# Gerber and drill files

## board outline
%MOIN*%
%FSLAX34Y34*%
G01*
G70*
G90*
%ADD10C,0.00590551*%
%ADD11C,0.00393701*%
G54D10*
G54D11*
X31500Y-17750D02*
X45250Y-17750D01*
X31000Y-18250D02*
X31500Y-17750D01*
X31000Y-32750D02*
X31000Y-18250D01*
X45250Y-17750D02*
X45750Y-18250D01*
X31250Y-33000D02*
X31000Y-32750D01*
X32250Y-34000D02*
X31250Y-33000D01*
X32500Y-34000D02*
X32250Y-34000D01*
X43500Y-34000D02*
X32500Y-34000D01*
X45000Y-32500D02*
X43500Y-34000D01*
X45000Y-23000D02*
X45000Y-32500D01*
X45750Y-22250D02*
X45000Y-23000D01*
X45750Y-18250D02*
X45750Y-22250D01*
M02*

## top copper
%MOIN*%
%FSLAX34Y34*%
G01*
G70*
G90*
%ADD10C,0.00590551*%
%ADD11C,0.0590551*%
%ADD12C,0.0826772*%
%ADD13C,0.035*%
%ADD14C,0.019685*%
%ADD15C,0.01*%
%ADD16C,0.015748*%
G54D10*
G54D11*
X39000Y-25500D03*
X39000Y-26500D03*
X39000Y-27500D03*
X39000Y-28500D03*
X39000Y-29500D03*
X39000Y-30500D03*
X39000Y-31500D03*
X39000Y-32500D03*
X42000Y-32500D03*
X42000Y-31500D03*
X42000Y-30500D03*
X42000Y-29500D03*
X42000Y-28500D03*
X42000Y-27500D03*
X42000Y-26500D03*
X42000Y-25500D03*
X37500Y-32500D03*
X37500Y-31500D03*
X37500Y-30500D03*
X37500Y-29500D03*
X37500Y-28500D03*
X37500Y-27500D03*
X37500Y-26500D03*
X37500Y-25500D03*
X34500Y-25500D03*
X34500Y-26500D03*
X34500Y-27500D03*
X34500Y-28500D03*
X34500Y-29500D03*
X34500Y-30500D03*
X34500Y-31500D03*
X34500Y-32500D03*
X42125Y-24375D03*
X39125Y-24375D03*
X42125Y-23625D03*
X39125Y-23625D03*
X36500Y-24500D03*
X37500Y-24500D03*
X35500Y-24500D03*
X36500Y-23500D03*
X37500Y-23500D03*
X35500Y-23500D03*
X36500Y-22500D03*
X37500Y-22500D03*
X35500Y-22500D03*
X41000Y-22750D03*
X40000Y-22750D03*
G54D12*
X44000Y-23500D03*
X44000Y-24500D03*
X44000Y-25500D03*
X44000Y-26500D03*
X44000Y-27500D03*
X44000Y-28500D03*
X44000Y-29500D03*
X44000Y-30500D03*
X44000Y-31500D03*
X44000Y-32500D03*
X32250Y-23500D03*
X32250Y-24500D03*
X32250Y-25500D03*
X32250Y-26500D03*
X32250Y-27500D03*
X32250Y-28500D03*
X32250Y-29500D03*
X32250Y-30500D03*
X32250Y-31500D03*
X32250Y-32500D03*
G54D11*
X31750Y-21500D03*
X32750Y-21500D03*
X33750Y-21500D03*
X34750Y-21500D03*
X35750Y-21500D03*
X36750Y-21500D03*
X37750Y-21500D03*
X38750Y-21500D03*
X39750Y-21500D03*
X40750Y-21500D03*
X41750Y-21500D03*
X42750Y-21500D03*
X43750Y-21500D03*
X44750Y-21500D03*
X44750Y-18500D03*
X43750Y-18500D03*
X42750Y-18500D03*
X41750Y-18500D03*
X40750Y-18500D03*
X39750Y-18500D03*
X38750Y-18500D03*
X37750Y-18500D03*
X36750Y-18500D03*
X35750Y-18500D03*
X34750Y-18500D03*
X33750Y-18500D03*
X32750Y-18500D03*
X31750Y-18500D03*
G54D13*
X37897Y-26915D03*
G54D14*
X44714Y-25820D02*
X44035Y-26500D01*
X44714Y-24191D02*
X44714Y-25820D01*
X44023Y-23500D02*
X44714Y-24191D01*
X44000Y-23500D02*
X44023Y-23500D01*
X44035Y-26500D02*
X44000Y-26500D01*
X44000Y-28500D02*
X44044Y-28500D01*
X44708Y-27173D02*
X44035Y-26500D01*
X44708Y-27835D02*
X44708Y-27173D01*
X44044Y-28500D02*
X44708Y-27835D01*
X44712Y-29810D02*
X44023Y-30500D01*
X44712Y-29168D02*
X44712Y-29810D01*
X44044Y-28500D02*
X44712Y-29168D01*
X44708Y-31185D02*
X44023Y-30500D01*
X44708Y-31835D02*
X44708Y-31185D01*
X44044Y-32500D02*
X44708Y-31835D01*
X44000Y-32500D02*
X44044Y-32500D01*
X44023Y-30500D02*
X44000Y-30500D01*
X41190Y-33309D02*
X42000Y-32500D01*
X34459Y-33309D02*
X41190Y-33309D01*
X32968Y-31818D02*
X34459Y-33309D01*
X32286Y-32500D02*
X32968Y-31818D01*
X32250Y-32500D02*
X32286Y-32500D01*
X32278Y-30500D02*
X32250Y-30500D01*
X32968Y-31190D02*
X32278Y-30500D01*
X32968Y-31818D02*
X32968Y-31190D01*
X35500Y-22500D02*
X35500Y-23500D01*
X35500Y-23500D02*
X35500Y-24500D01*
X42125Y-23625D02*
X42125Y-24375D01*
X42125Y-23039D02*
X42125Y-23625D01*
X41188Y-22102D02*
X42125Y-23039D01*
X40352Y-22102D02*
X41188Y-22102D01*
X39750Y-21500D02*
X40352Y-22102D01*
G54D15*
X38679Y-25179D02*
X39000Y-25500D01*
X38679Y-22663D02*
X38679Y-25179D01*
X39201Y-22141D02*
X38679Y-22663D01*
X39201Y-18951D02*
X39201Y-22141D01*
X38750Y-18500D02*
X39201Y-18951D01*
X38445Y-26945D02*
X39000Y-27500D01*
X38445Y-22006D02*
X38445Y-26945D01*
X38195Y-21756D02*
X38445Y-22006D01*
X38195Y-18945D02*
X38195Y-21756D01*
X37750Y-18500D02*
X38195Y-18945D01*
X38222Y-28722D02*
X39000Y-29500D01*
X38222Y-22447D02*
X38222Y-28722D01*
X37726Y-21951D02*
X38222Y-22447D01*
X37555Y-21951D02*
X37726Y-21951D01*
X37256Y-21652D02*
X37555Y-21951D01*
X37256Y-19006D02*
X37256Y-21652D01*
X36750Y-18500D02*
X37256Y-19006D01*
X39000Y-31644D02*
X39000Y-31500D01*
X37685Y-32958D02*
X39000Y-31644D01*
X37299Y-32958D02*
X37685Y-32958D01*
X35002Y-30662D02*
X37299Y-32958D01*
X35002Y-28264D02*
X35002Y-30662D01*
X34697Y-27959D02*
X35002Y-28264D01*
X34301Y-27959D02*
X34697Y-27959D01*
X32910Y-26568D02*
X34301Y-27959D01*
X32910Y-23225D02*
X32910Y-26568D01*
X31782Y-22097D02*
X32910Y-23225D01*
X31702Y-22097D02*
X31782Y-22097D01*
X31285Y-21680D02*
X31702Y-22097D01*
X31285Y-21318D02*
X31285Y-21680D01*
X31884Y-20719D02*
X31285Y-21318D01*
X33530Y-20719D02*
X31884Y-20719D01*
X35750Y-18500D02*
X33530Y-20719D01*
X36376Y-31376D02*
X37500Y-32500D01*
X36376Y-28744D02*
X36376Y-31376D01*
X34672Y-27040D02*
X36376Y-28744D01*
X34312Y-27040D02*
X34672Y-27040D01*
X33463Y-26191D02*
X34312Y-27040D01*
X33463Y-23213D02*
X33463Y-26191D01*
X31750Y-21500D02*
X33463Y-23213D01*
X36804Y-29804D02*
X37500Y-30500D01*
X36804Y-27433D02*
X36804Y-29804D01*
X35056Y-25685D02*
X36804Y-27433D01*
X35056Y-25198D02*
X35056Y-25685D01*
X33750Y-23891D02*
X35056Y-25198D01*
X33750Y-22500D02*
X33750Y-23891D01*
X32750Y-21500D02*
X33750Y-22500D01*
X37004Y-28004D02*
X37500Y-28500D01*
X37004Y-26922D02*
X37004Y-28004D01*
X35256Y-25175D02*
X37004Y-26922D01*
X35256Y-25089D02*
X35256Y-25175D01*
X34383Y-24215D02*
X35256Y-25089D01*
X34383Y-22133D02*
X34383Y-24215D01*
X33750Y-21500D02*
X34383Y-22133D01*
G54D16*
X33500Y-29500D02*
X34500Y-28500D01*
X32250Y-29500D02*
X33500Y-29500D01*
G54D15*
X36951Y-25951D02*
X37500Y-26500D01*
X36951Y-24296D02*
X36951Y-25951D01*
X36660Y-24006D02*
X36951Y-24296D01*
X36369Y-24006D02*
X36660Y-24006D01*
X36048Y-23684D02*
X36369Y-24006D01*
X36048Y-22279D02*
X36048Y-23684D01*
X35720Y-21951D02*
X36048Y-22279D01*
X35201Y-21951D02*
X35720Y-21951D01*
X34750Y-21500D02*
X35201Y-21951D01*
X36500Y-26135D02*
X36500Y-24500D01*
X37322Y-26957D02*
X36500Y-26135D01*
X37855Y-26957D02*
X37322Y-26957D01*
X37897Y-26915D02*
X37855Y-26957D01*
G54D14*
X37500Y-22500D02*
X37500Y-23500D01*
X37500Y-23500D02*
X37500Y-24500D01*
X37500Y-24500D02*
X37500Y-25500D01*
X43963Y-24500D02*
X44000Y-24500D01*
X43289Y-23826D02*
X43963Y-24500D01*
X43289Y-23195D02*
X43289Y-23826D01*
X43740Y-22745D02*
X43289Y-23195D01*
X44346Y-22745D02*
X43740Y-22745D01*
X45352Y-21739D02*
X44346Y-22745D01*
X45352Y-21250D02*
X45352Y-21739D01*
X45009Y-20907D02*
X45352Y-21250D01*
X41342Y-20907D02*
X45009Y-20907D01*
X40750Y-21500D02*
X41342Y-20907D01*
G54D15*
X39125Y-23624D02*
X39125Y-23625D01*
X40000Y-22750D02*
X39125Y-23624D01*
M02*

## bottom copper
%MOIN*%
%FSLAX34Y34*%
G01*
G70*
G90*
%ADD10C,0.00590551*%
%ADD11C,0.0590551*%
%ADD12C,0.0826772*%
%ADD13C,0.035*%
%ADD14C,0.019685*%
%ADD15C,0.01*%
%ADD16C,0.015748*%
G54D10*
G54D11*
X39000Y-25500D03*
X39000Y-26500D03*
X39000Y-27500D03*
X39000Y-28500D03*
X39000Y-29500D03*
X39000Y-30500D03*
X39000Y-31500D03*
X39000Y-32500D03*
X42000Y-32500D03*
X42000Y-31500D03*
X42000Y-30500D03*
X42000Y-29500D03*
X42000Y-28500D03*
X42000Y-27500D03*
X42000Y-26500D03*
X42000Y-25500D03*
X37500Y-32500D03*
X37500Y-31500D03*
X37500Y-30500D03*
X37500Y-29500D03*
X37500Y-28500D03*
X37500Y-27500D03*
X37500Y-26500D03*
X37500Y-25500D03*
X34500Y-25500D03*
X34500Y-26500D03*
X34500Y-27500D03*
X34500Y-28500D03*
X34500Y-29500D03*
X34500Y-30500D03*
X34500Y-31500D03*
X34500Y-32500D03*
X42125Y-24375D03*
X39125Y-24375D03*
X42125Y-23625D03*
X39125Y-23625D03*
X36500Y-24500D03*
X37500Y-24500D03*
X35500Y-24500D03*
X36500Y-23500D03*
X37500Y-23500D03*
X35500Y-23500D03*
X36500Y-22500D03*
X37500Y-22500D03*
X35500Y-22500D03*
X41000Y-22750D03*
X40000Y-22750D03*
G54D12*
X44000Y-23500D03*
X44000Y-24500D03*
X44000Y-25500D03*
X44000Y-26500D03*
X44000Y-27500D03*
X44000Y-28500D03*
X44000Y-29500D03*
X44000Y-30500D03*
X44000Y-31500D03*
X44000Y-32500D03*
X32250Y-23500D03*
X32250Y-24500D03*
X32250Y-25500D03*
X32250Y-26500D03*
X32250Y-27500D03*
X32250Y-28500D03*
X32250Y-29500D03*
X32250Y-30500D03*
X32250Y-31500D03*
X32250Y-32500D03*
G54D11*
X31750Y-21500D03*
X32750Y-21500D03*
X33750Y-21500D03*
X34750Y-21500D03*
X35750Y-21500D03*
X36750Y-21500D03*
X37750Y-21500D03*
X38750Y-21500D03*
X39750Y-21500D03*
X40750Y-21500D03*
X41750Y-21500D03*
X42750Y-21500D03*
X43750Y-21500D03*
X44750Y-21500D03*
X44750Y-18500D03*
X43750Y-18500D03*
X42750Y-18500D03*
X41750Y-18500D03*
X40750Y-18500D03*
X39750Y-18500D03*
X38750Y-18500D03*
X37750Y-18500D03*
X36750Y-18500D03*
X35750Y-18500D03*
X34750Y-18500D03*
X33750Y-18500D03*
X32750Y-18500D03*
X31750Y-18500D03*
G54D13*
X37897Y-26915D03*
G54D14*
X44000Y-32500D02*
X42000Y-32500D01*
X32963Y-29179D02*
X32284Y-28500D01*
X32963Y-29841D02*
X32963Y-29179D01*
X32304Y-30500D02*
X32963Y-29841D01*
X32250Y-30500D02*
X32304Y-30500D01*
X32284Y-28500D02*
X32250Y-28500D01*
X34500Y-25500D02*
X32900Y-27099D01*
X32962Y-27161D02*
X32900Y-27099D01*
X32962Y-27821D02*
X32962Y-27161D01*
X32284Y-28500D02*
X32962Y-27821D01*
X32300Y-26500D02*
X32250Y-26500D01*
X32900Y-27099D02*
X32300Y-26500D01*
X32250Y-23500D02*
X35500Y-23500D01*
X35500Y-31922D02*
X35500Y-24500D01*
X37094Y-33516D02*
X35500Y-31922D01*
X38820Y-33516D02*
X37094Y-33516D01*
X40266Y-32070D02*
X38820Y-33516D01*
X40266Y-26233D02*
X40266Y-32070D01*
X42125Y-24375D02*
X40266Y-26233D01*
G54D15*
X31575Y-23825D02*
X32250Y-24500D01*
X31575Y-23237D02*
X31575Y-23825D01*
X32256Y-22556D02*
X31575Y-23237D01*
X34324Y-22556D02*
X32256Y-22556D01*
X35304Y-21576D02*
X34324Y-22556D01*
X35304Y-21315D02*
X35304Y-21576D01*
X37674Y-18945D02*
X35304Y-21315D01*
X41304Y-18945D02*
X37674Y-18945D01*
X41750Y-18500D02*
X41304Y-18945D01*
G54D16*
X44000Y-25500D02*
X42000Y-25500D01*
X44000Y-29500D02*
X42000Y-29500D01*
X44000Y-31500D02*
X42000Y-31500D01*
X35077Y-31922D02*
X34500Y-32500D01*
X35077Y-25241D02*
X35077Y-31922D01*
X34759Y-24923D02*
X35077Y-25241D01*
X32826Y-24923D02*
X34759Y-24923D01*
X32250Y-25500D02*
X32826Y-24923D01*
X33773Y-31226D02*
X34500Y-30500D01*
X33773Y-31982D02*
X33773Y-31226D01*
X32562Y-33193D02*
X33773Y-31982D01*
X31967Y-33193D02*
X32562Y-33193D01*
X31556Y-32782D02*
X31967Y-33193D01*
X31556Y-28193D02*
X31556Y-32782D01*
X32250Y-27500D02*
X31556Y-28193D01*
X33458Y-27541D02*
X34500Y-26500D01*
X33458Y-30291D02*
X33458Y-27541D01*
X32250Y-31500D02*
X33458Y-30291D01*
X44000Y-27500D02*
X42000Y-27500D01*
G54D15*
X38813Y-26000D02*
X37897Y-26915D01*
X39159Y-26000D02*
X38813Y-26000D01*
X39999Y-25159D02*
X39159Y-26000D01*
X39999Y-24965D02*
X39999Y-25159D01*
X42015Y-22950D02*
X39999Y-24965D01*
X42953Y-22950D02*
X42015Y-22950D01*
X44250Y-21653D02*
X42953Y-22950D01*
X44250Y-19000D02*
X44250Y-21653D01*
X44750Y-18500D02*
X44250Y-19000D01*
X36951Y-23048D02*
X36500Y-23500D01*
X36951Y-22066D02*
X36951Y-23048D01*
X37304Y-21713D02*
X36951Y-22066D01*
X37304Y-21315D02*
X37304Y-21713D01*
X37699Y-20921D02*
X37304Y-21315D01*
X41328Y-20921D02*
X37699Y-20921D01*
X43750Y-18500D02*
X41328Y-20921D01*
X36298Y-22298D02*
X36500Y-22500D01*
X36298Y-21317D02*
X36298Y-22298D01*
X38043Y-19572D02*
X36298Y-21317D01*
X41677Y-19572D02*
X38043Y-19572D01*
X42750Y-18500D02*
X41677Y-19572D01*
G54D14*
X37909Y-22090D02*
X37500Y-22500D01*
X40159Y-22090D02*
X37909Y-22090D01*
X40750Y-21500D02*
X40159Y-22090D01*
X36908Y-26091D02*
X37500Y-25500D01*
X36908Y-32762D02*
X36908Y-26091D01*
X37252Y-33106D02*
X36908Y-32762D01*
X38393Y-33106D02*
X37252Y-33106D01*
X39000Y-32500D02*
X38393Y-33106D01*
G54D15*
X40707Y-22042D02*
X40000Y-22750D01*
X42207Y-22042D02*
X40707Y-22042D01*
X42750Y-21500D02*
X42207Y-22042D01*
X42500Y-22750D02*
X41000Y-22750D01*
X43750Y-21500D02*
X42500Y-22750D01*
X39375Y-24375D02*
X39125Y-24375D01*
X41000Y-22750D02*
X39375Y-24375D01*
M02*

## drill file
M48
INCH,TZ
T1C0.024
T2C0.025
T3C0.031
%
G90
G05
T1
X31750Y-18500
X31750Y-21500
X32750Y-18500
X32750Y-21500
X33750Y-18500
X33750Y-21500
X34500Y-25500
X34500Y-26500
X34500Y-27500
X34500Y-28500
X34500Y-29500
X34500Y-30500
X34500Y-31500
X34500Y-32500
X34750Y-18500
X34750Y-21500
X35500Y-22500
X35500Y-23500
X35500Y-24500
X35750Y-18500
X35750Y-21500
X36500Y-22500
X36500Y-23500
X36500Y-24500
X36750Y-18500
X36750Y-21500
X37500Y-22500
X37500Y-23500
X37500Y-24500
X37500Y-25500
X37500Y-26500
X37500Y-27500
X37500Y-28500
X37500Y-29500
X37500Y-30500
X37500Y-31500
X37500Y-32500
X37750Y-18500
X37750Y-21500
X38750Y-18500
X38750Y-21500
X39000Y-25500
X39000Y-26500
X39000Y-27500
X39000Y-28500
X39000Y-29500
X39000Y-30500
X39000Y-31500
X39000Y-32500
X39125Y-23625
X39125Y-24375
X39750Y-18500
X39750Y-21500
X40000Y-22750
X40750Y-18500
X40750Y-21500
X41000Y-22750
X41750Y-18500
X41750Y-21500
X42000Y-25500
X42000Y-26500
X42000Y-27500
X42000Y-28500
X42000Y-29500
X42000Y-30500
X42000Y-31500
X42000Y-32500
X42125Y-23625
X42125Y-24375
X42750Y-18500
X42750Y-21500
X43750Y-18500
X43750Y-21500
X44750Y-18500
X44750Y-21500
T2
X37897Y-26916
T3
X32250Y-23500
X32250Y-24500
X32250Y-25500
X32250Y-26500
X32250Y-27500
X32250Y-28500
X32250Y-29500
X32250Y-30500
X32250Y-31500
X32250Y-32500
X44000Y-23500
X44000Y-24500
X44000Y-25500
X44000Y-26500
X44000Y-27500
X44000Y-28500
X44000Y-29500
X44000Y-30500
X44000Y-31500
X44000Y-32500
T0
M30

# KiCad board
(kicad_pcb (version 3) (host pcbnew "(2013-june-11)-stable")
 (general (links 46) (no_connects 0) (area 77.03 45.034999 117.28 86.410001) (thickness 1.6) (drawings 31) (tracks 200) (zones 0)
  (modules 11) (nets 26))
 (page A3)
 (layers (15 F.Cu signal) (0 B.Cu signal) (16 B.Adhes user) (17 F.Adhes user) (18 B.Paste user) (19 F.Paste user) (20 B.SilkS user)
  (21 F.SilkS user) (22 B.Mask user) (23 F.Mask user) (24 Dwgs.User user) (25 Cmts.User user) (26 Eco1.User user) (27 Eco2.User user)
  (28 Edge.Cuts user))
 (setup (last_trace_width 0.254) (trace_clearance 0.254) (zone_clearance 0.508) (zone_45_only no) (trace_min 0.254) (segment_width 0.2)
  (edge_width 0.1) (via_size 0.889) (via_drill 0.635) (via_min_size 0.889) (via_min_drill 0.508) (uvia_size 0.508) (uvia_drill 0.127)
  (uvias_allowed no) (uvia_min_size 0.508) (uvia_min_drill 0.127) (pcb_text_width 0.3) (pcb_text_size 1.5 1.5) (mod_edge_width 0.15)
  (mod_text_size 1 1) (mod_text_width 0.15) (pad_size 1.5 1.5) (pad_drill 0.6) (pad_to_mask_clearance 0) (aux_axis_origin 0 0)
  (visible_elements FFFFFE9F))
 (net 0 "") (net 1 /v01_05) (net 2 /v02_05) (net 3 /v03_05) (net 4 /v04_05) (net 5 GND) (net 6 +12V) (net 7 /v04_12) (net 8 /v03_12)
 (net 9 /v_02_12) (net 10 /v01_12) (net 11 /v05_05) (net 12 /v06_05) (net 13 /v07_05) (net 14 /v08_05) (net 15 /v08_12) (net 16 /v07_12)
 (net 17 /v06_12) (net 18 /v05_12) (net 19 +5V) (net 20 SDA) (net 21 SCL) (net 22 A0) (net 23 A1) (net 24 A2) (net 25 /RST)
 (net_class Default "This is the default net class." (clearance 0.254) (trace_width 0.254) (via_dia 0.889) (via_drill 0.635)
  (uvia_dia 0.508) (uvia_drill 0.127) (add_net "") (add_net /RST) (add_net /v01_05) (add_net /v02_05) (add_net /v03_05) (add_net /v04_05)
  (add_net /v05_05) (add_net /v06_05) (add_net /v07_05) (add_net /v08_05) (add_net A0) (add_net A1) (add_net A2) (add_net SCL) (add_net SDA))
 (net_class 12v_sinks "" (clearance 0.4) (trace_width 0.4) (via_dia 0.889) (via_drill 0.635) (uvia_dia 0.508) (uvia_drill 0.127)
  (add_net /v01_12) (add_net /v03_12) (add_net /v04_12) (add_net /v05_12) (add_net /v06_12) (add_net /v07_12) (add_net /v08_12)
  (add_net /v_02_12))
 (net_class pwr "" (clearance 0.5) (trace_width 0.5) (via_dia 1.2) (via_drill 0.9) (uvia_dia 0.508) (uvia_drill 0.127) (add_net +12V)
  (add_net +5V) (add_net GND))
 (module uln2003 (layer F.Cu) (at 100.33 74.93)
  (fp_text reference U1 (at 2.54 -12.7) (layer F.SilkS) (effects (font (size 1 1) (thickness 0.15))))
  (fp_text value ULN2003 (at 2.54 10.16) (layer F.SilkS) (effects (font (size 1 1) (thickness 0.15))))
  (pad 1 thru_hole circle (at -1.27 -10.16) (size 1.5 1.5) (drill 0.6) (layers *.Cu *.Mask F.SilkS) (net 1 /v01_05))
  (pad 2 thru_hole circle (at -1.27 -7.62) (size 1.5 1.5) (drill 0.6) (layers *.Cu *.Mask F.SilkS))
  (pad 3 thru_hole circle (at -1.27 -5.08) (size 1.5 1.5) (drill 0.6) (layers *.Cu *.Mask F.SilkS) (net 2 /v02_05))
  (pad 4 thru_hole circle (at -1.27 -2.54) (size 1.5 1.5) (drill 0.6) (layers *.Cu *.Mask F.SilkS))
  (pad 5 thru_hole circle (at -1.27 0) (size 1.5 1.5) (drill 0.6) (layers *.Cu *.Mask F.SilkS) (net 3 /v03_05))
  (pad 6 thru_hole circle (at -1.27 2.54) (size 1.5 1.5) (drill 0.6) (layers *.Cu *.Mask F.SilkS))
  (pad 7 thru_hole circle (at -1.27 5.08) (size 1.5 1.5) (drill 0.6) (layers *.Cu *.Mask F.SilkS) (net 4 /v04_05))
  (pad 8 thru_hole circle (at -1.27 7.62) (size 1.5 1.5) (drill 0.6) (layers *.Cu *.Mask F.SilkS) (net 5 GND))
  (pad 9 thru_hole circle (at 6.35 7.62) (size 1.5 1.5) (drill 0.6) (layers *.Cu *.Mask F.SilkS) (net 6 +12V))
  (pad 10 thru_hole circle (at 6.35 5.08) (size 1.5 1.5) (drill 0.6) (layers *.Cu *.Mask F.SilkS) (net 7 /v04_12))
  (pad 11 thru_hole circle (at 6.35 2.54) (size 1.5 1.5) (drill 0.6) (layers *.Cu *.Mask F.SilkS))
  (pad 12 thru_hole circle (at 6.35 0) (size 1.5 1.5) (drill 0.6) (layers *.Cu *.Mask F.SilkS) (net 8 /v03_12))
  (pad 13 thru_hole circle (at 6.35 -2.54) (size 1.5 1.5) (drill 0.6) (layers *.Cu *.Mask F.SilkS))
  (pad 14 thru_hole circle (at 6.35 -5.08) (size 1.5 1.5) (drill 0.6) (layers *.Cu *.Mask F.SilkS) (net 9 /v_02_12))
  (pad 15 thru_hole circle (at 6.35 -7.62) (size 1.5 1.5) (drill 0.6) (layers *.Cu *.Mask F.SilkS))
  (pad 16 thru_hole circle (at 6.35 -10.16) (size 1.5 1.5) (drill 0.6) (layers *.Cu *.Mask F.SilkS) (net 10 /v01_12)))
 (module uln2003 (layer F.Cu) (at 93.98 72.39 180)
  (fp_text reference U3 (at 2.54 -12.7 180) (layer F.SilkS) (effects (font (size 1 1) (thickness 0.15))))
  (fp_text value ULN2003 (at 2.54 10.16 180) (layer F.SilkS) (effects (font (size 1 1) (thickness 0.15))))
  (pad 1 thru_hole circle (at -1.27 -10.16 180) (size 1.5 1.5) (drill 0.6) (layers *.Cu *.Mask F.SilkS) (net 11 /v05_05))
  (pad 2 thru_hole circle (at -1.27 -7.62 180) (size 1.5 1.5) (drill 0.6) (layers *.Cu *.Mask F.SilkS))
  (pad 3 thru_hole circle (at -1.27 -5.08 180) (size 1.5 1.5) (drill 0.6) (layers *.Cu *.Mask F.SilkS) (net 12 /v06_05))
  (pad 4 thru_hole circle (at -1.27 -2.54 180) (size 1.5 1.5) (drill 0.6) (layers *.Cu *.Mask F.SilkS))
  (pad 5 thru_hole circle (at -1.27 0 180) (size 1.5 1.5) (drill 0.6) (layers *.Cu *.Mask F.SilkS) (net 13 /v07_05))
  (pad 6 thru_hole circle (at -1.27 2.54 180) (size 1.5 1.5) (drill 0.6) (layers *.Cu *.Mask F.SilkS))
  (pad 7 thru_hole circle (at -1.27 5.08 180) (size 1.5 1.5) (drill 0.6) (layers *.Cu *.Mask F.SilkS) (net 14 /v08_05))
  (pad 8 thru_hole circle (at -1.27 7.62 180) (size 1.5 1.5) (drill 0.6) (layers *.Cu *.Mask F.SilkS) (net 5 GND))
  (pad 9 thru_hole circle (at 6.35 7.62 180) (size 1.5 1.5) (drill 0.6) (layers *.Cu *.Mask F.SilkS) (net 6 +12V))
  (pad 10 thru_hole circle (at 6.35 5.08 180) (size 1.5 1.5) (drill 0.6) (layers *.Cu *.Mask F.SilkS) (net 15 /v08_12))
  (pad 11 thru_hole circle (at 6.35 2.54 180) (size 1.5 1.5) (drill 0.6) (layers *.Cu *.Mask F.SilkS))
  (pad 12 thru_hole circle (at 6.35 0 180) (size 1.5 1.5) (drill 0.6) (layers *.Cu *.Mask F.SilkS) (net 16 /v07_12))
  (pad 13 thru_hole circle (at 6.35 -2.54 180) (size 1.5 1.5) (drill 0.6) (layers *.Cu *.Mask F.SilkS))
  (pad 14 thru_hole circle (at 6.35 -5.08 180) (size 1.5 1.5) (drill 0.6) (layers *.Cu *.Mask F.SilkS) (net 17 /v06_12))
  (pad 15 thru_hole circle (at 6.35 -7.62 180) (size 1.5 1.5) (drill 0.6) (layers *.Cu *.Mask F.SilkS))
  (pad 16 thru_hole circle (at 6.35 -10.16 180) (size 1.5 1.5) (drill 0.6) (layers *.Cu *.Mask F.SilkS) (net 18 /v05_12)))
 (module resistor (layer F.Cu) (at 104.458 61.9125 180)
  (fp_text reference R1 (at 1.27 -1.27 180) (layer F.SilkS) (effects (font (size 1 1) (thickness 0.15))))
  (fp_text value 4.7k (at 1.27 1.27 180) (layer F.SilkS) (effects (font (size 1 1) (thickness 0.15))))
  (pad 1 thru_hole circle (at -2.54 0 180) (size 1.5 1.5) (drill 0.6) (layers *.Cu *.Mask F.SilkS) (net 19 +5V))
  (pad 2 thru_hole circle (at 5.08 0 180) (size 1.5 1.5) (drill 0.6) (layers *.Cu *.Mask F.SilkS) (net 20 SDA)))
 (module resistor (layer F.Cu) (at 104.458 60.0075 180)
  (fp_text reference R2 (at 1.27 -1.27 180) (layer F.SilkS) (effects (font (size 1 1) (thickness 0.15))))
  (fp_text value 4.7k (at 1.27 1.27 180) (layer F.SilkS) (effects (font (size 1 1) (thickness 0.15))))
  (pad 1 thru_hole circle (at -2.54 0 180) (size 1.5 1.5) (drill 0.6) (layers *.Cu *.Mask F.SilkS) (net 19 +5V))
  (pad 2 thru_hole circle (at 5.08 0 180) (size 1.5 1.5) (drill 0.6) (layers *.Cu *.Mask F.SilkS) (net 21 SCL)))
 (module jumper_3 (layer F.Cu) (at 92.71 62.23)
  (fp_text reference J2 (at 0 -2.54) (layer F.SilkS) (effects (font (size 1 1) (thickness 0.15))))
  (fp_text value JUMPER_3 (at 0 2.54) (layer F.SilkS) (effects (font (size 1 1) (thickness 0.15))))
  (pad 2 thru_hole circle (at 0 0) (size 1.5 1.5) (drill 0.6) (layers *.Cu *.Mask F.SilkS) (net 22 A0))
  (pad 3 thru_hole circle (at 2.54 0) (size 1.5 1.5) (drill 0.6) (layers *.Cu *.Mask F.SilkS) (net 5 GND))
  (pad 1 thru_hole circle (at -2.54 0) (size 1.5 1.5) (drill 0.6) (layers *.Cu *.Mask F.SilkS) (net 19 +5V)))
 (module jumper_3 (layer F.Cu) (at 92.71 59.69)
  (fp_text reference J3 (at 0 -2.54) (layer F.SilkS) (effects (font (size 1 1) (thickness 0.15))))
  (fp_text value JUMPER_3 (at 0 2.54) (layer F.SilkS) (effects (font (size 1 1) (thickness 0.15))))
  (pad 2 thru_hole circle (at 0 0) (size 1.5 1.5) (drill 0.6) (layers *.Cu *.Mask F.SilkS) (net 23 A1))
  (pad 3 thru_hole circle (at 2.54 0) (size 1.5 1.5) (drill 0.6) (layers *.Cu *.Mask F.SilkS) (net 5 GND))
  (pad 1 thru_hole circle (at -2.54 0) (size 1.5 1.5) (drill 0.6) (layers *.Cu *.Mask F.SilkS) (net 19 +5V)))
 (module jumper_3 (layer F.Cu) (at 92.71 57.15)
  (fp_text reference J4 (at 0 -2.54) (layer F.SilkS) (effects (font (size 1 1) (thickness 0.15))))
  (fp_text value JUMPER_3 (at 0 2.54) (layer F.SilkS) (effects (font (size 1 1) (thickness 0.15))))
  (pad 2 thru_hole circle (at 0 0) (size 1.5 1.5) (drill 0.6) (layers *.Cu *.Mask F.SilkS) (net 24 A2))
  (pad 3 thru_hole circle (at 2.54 0) (size 1.5 1.5) (drill 0.6) (layers *.Cu *.Mask F.SilkS) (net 5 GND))
  (pad 1 thru_hole circle (at -2.54 0) (size 1.5 1.5) (drill 0.6) (layers *.Cu *.Mask F.SilkS) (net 19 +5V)))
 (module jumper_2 (layer F.Cu) (at 102.87 57.785 180)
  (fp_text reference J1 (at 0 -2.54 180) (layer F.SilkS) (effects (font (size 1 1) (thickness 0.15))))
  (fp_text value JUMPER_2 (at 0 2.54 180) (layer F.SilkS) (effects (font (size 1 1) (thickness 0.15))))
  (pad 1 thru_hole circle (at -1.27 0 180) (size 1.5 1.5) (drill 0.6) (layers *.Cu *.Mask F.SilkS) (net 20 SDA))
  (pad 2 thru_hole circle (at 1.27 0 180) (size 1.5 1.5) (drill 0.6) (layers *.Cu *.Mask F.SilkS) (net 21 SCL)))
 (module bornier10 (layer F.Cu) (at 111.76 72.39 270)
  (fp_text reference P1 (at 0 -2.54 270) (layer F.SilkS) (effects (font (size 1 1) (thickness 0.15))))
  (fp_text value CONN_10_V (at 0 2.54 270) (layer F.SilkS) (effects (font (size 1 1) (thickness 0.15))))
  (pad 1 thru_hole circle (at -12.7 0 270) (size 2.1 2.1) (drill 0.8) (layers *.Cu *.Mask F.SilkS) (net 6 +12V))
  (pad 2 thru_hole circle (at -10.16 0 270) (size 2.1 2.1) (drill 0.8) (layers *.Cu *.Mask F.SilkS) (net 5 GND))
  (pad 3 thru_hole circle (at -7.62 0 270) (size 2.1 2.1) (drill 0.8) (layers *.Cu *.Mask F.SilkS) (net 10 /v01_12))
  (pad 4 thru_hole circle (at -5.08 0 270) (size 2.1 2.1) (drill 0.8) (layers *.Cu *.Mask F.SilkS) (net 6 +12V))
  (pad 5 thru_hole circle (at -2.54 0 270) (size 2.1 2.1) (drill 0.8) (layers *.Cu *.Mask F.SilkS) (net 9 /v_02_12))
  (pad 6 thru_hole circle (at 0 0 270) (size 2.1 2.1) (drill 0.8) (layers *.Cu *.Mask F.SilkS) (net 6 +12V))
  (pad 7 thru_hole circle (at 2.54 0 270) (size 2.1 2.1) (drill 0.8) (layers *.Cu *.Mask F.SilkS) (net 8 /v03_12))
  (pad 8 thru_hole circle (at 5.08 0 270) (size 2.1 2.1) (drill 0.8) (layers *.Cu *.Mask F.SilkS) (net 6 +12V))
  (pad 9 thru_hole circle (at 7.62 0 270) (size 2.1 2.1) (drill 0.8) (layers *.Cu *.Mask F.SilkS) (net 7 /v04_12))
  (pad 10 thru_hole circle (at 10.16 0 270) (size 2.1 2.1) (drill 0.8) (layers *.Cu *.Mask F.SilkS) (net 6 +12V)))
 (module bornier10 (layer F.Cu) (at 81.915 72.39 270)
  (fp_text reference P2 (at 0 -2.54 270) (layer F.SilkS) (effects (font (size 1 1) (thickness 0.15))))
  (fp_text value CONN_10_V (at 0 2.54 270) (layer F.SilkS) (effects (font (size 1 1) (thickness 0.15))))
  (pad 1 thru_hole circle (at -12.7 0 270) (size 2.1 2.1) (drill 0.8) (layers *.Cu *.Mask F.SilkS) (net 19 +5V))
  (pad 2 thru_hole circle (at -10.16 0 270) (size 2.1 2.1) (drill 0.8) (layers *.Cu *.Mask F.SilkS) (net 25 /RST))
  (pad 3 thru_hole circle (at -7.62 0 270) (size 2.1 2.1) (drill 0.8) (layers *.Cu *.Mask F.SilkS) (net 18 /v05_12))
  (pad 4 thru_hole circle (at -5.08 0 270) (size 2.1 2.1) (drill 0.8) (layers *.Cu *.Mask F.SilkS) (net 6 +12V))
  (pad 5 thru_hole circle (at -2.54 0 270) (size 2.1 2.1) (drill 0.8) (layers *.Cu *.Mask F.SilkS) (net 17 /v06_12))
  (pad 6 thru_hole circle (at 0 0 270) (size 2.1 2.1) (drill 0.8) (layers *.Cu *.Mask F.SilkS) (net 6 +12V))
  (pad 7 thru_hole circle (at 2.54 0 270) (size 2.1 2.1) (drill 0.8) (layers *.Cu *.Mask F.SilkS) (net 16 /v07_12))
  (pad 8 thru_hole circle (at 5.08 0 270) (size 2.1 2.1) (drill 0.8) (layers *.Cu *.Mask F.SilkS) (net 6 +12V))
  (pad 9 thru_hole circle (at 7.62 0 270) (size 2.1 2.1) (drill 0.8) (layers *.Cu *.Mask F.SilkS) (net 15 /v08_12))
  (pad 10 thru_hole circle (at 10.16 0 270) (size 2.1 2.1) (drill 0.8) (layers *.Cu *.Mask F.SilkS) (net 6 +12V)))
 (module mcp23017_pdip (layer F.Cu) (at 93.345 53.34 90)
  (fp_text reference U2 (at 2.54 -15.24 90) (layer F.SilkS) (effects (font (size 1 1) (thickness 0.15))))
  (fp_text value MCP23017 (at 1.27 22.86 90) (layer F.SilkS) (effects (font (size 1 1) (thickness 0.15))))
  (pad 1 thru_hole circle (at -1.27 -12.7 90) (size 1.5 1.5) (drill 0.6) (layers *.Cu *.Mask F.SilkS) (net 11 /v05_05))
  (pad 2 thru_hole circle (at -1.27 -10.16 90) (size 1.5 1.5) (drill 0.6) (layers *.Cu *.Mask F.SilkS) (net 12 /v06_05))
  (pad 3 thru_hole circle (at -1.27 -7.62 90) (size 1.5 1.5) (drill 0.6) (layers *.Cu *.Mask F.SilkS) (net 13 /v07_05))
  (pad 4 thru_hole circle (at -1.27 -5.08 90) (size 1.5 1.5) (drill 0.6) (layers *.Cu *.Mask F.SilkS) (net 14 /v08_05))
  (pad 5 thru_hole circle (at -1.27 -2.54 90) (size 1.5 1.5) (drill 0.6) (layers *.Cu *.Mask F.SilkS))
  (pad 6 thru_hole circle (at -1.27 0 90) (size 1.5 1.5) (drill 0.6) (layers *.Cu *.Mask F.SilkS))
  (pad 7 thru_hole circle (at -1.27 2.54 90) (size 1.5 1.5) (drill 0.6) (layers *.Cu *.Mask F.SilkS))
  (pad 8 thru_hole circle (at -1.27 5.08 90) (size 1.5 1.5) (drill 0.6) (layers *.Cu *.Mask F.SilkS))
  (pad 9 thru_hole circle (at -1.27 7.62 90) (size 1.5 1.5) (drill 0.6) (layers *.Cu *.Mask F.SilkS) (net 19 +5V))
  (pad 10 thru_hole circle (at -1.27 10.16 90) (size 1.5 1.5) (drill 0.6) (layers *.Cu *.Mask F.SilkS) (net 5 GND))
  (pad 11 thru_hole circle (at -1.27 12.7 90) (size 1.5 1.5) (drill 0.6) (layers *.Cu *.Mask F.SilkS))
  (pad 12 thru_hole circle (at -1.27 15.24 90) (size 1.5 1.5) (drill 0.6) (layers *.Cu *.Mask F.SilkS) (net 21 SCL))
  (pad 13 thru_hole circle (at -1.27 17.78 90) (size 1.5 1.5) (drill 0.6) (layers *.Cu *.Mask F.SilkS) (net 20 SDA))
  (pad 14 thru_hole circle (at -1.27 20.32 90) (size 1.5 1.5) (drill 0.6) (layers *.Cu *.Mask F.SilkS))
  (pad 15 thru_hole circle (at 6.35 20.32 90) (size 1.5 1.5) (drill 0.6) (layers *.Cu *.Mask F.SilkS) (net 22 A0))
  (pad 16 thru_hole circle (at 6.35 17.78 90) (size 1.5 1.5) (drill 0.6) (layers *.Cu *.Mask F.SilkS) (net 23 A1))
  (pad 17 thru_hole circle (at 6.35 15.24 90) (size 1.5 1.5) (drill 0.6) (layers *.Cu *.Mask F.SilkS) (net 24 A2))
  (pad 18 thru_hole circle (at 6.35 12.7 90) (size 1.5 1.5) (drill 0.6) (layers *.Cu *.Mask F.SilkS) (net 25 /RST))
  (pad 19 thru_hole circle (at 6.35 10.16 90) (size 1.5 1.5) (drill 0.6) (layers *.Cu *.Mask F.SilkS))
  (pad 20 thru_hole circle (at 6.35 7.62 90) (size 1.5 1.5) (drill 0.6) (layers *.Cu *.Mask F.SilkS))
  (pad 21 thru_hole circle (at 6.35 5.08 90) (size 1.5 1.5) (drill 0.6) (layers *.Cu *.Mask F.SilkS) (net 1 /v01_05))
  (pad 22 thru_hole circle (at 6.35 2.54 90) (size 1.5 1.5) (drill 0.6) (layers *.Cu *.Mask F.SilkS) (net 2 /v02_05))
  (pad 23 thru_hole circle (at 6.35 0 90) (size 1.5 1.5) (drill 0.6) (layers *.Cu *.Mask F.SilkS) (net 3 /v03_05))
  (pad 24 thru_hole circle (at 6.35 -2.54 90) (size 1.5 1.5) (drill 0.6) (layers *.Cu *.Mask F.SilkS) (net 4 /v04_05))
  (pad 25 thru_hole circle (at 6.35 -5.08 90) (size 1.5 1.5) (drill 0.6) (layers *.Cu *.Mask F.SilkS))
  (pad 26 thru_hole circle (at 6.35 -7.62 90) (size 1.5 1.5) (drill 0.6) (layers *.Cu *.Mask F.SilkS))
  (pad 27 thru_hole circle (at 6.35 -10.16 90) (size 1.5 1.5) (drill 0.6) (layers *.Cu *.Mask F.SilkS))
  (pad 28 thru_hole circle (at 6.35 -12.7 90) (size 1.5 1.5) (drill 0.6) (layers *.Cu *.Mask F.SilkS)))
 (gr_line (start 80.01 45.085) (end 114.935 45.085) (angle 90) (layer Edge.Cuts) (width 0.1))
 (gr_line (start 78.74 46.355) (end 80.01 45.085) (angle 90) (layer Edge.Cuts) (width 0.1))
 (gr_line (start 78.74 83.185) (end 78.74 46.355) (angle 90) (layer Edge.Cuts) (width 0.1))
 (gr_line (start 114.935 45.085) (end 116.205 46.355) (angle 90) (layer Edge.Cuts) (width 0.1))
 (gr_line (start 79.375 83.82) (end 78.74 83.185) (angle 90) (layer Edge.Cuts) (width 0.1))
 (gr_line (start 81.915 86.36) (end 79.375 83.82) (angle 90) (layer Edge.Cuts) (width 0.1))
 (gr_line (start 82.55 86.36) (end 81.915 86.36) (angle 90) (layer Edge.Cuts) (width 0.1))
 (gr_line (start 110.49 86.36) (end 82.55 86.36) (angle 90) (layer Edge.Cuts) (width 0.1))
 (gr_line (start 114.3 82.55) (end 110.49 86.36) (angle 90) (layer Edge.Cuts) (width 0.1))
 (gr_line (start 114.3 58.42) (end 114.3 82.55) (angle 90) (layer Edge.Cuts) (width 0.1))
 (gr_line (start 116.205 56.515) (end 114.3 58.42) (angle 90) (layer Edge.Cuts) (width 0.1))
 (gr_line (start 116.205 46.355) (end 116.205 56.515) (angle 90) (layer Edge.Cuts) (width 0.1))
 (segment (start 111.76 82.55) (end 106.68 82.55) (width 0.5) (layer B.Cu) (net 6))
 (segment (start 113.5758 65.5848) (end 111.8506 67.31) (width 0.5) (layer F.Cu) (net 6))
 (segment (start 113.5758 61.4456) (end 113.5758 65.5848) (width 0.5) (layer F.Cu) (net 6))
 (segment (start 111.8202 59.69) (end 113.5758 61.4456) (width 0.5) (layer F.Cu) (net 6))
 (segment (start 111.76 59.69) (end 111.8202 59.69) (width 0.5) (layer F.Cu) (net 6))
 (segment (start 111.8506 67.31) (end 111.76 67.31) (width 0.5) (layer F.Cu) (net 6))
 (segment (start 111.76 72.39) (end 111.8727 72.39) (width 0.5) (layer F.Cu) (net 6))
 (segment (start 113.5604 69.0198) (end 111.8506 67.31) (width 0.5) (layer F.Cu) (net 6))
 (segment (start 113.5604 70.7023) (end 113.5604 69.0198) (width 0.5) (layer F.Cu) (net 6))
 (segment (start 111.8727 72.39) (end 113.5604 70.7023) (width 0.5) (layer F.Cu) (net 6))
 (segment (start 113.5707 75.7195) (end 111.8202 77.47) (width 0.5) (layer F.Cu) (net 6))
 (segment (start 113.5707 74.088) (end 113.5707 75.7195) (width 0.5) (layer F.Cu) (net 6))
 (segment (start 111.8727 72.39) (end 113.5707 74.088) (width 0.5) (layer F.Cu) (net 6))
 (segment (start 113.5604 79.2102) (end 111.8202 77.47) (width 0.5) (layer F.Cu) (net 6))
 (segment (start 113.5604 80.862) (end 113.5604 79.2102) (width 0.5) (layer F.Cu) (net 6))
 (segment (start 111.8724 82.55) (end 113.5604 80.862) (width 0.5) (layer F.Cu) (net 6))
 (segment (start 111.76 82.55) (end 111.8724 82.55) (width 0.5) (layer F.Cu) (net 6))
 (segment (start 111.8202 77.47) (end 111.76 77.47) (width 0.5) (layer F.Cu) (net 6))
 (segment (start 83.7261 74.1147) (end 82.0014 72.39) (width 0.5) (layer B.Cu) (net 6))
 (segment (start 83.7261 75.7966) (end 83.7261 74.1147) (width 0.5) (layer B.Cu) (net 6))
 (segment (start 82.0527 77.47) (end 83.7261 75.7966) (width 0.5) (layer B.Cu) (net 6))
 (segment (start 81.915 77.47) (end 82.0527 77.47) (width 0.5) (layer B.Cu) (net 6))
 (segment (start 82.0014 72.39) (end 81.915 72.39) (width 0.5) (layer B.Cu) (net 6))
 (segment (start 87.63 64.77) (end 83.5668 68.8332) (width 0.5) (layer B.Cu) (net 6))
 (segment (start 83.7246 68.9911) (end 83.5668 68.8332) (width 0.5) (layer B.Cu) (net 6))
 (segment (start 83.7246 70.6668) (end 83.7246 68.9911) (width 0.5) (layer B.Cu) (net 6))
 (segment (start 82.0014 72.39) (end 83.7246 70.6668) (width 0.5) (layer B.Cu) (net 6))
 (segment (start 82.0435 67.31) (end 81.915 67.31) (width 0.5) (layer B.Cu) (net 6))
 (segment (start 83.5668 68.8332) (end 82.0435 67.31) (width 0.5) (layer B.Cu) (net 6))
 (segment (start 104.6234 84.6066) (end 106.68 82.55) (width 0.5) (layer F.Cu) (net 6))
 (segment (start 87.5283 84.6066) (end 104.6234 84.6066) (width 0.5) (layer F.Cu) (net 6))
 (segment (start 83.74 80.8183) (end 87.5283 84.6066) (width 0.5) (layer F.Cu) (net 6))
 (segment (start 82.0083 82.55) (end 83.74 80.8183) (width 0.5) (layer F.Cu) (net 6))
 (segment (start 81.915 82.55) (end 82.0083 82.55) (width 0.5) (layer F.Cu) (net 6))
 (segment (start 81.9867 77.47) (end 81.915 77.47) (width 0.5) (layer F.Cu) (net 6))
 (segment (start 83.74 79.2233) (end 81.9867 77.47) (width 0.5) (layer F.Cu) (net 6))
 (segment (start 83.74 80.8183) (end 83.74 79.2233) (width 0.5) (layer F.Cu) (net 6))
 (segment (start 90.17 57.15) (end 90.17 59.69) (width 0.5) (layer F.Cu) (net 19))
 (segment (start 90.17 59.69) (end 90.17 62.23) (width 0.5) (layer F.Cu) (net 19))
 (segment (start 106.998 60.0075) (end 106.998 61.9125) (width 0.5) (layer F.Cu) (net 19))
 (segment (start 81.915 59.69) (end 90.17 59.69) (width 0.5) (layer B.Cu) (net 19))
 (segment (start 106.998 58.5203) (end 106.998 60.0075) (width 0.5) (layer F.Cu) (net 19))
 (segment (start 104.6186 56.1409) (end 106.998 58.5203) (width 0.5) (layer F.Cu) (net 19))
 (segment (start 102.4959 56.1409) (end 104.6186 56.1409) (width 0.5) (layer F.Cu) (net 19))
 (segment (start 100.965 54.61) (end 102.4959 56.1409) (width 0.5) (layer F.Cu) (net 19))
 (segment (start 90.17 81.0828) (end 90.17 62.23) (width 0.5) (layer B.Cu) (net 19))
 (segment (start 94.219 85.1318) (end 90.17 81.0828) (width 0.5) (layer B.Cu) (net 19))
 (segment (start 98.605 85.1318) (end 94.219 85.1318) (width 0.5) (layer B.Cu) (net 19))
 (segment (start 102.2779 81.4589) (end 98.605 85.1318) (width 0.5) (layer B.Cu) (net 19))
 (segment (start 102.2779 66.6326) (end 102.2779 81.4589) (width 0.5) (layer B.Cu) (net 19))
 (segment (start 106.998 61.9125) (end 102.2779 66.6326) (width 0.5) (layer B.Cu) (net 19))
 (segment (start 80.2013 60.5163) (end 81.915 62.23) (width 0.254) (layer B.Cu) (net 25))
 (segment (start 80.2013 59.0234) (end 80.2013 60.5163) (width 0.254) (layer B.Cu) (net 25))
 (segment (start 81.9309 57.2938) (end 80.2013 59.0234) (width 0.254) (layer B.Cu) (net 25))
 (segment (start 87.1848 57.2938) (end 81.9309 57.2938) (width 0.254) (layer B.Cu) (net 25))
 (segment (start 89.6736 54.805) (end 87.1848 57.2938) (width 0.254) (layer B.Cu) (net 25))
 (segment (start 89.6736 54.1415) (end 89.6736 54.805) (width 0.254) (layer B.Cu) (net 25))
 (segment (start 95.6937 48.1214) (end 89.6736 54.1415) (width 0.254) (layer B.Cu) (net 25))
 (segment (start 104.9136 48.1214) (end 95.6937 48.1214) (width 0.254) (layer B.Cu) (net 25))
 (segment (start 106.045 46.99) (end 104.9136 48.1214) (width 0.254) (layer B.Cu) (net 25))
 (segment (start 98.246 63.956) (end 99.06 64.77) (width 0.254) (layer F.Cu) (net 1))
 (segment (start 98.246 57.5663) (end 98.246 63.956) (width 0.254) (layer F.Cu) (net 1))
 (segment (start 99.572 56.2403) (end 98.246 57.5663) (width 0.254) (layer F.Cu) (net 1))
 (segment (start 99.572 48.137) (end 99.572 56.2403) (width 0.254) (layer F.Cu) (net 1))
 (segment (start 98.425 46.99) (end 99.572 48.137) (width 0.254) (layer F.Cu) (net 1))
 (segment (start 111.76 64.77) (end 106.68 64.77) (width 0.4) (layer B.Cu) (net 10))
 (segment (start 97.6514 68.4414) (end 99.06 69.85) (width 0.254) (layer F.Cu) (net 2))
 (segment (start 97.6514 55.8962) (end 97.6514 68.4414) (width 0.254) (layer F.Cu) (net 2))
 (segment (start 97.0164 55.2612) (end 97.6514 55.8962) (width 0.254) (layer F.Cu) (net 2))
 (segment (start 97.0164 48.1214) (end 97.0164 55.2612) (width 0.254) (layer F.Cu) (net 2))
 (segment (start 95.885 46.99) (end 97.0164 48.1214) (width 0.254) (layer F.Cu) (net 2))
 (segment (start 97.0852 72.9552) (end 99.06 74.93) (width 0.254) (layer F.Cu) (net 3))
 (segment (start 97.0852 57.0175) (end 97.0852 72.9552) (width 0.254) (layer F.Cu) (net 3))
 (segment (start 95.8247 55.757) (end 97.0852 57.0175) (width 0.254) (layer F.Cu) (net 3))
 (segment (start 95.3901 55.757) (end 95.8247 55.757) (width 0.254) (layer F.Cu) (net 3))
 (segment (start 94.6306 54.9975) (end 95.3901 55.757) (width 0.254) (layer F.Cu) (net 3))
 (segment (start 94.6306 48.2756) (end 94.6306 54.9975) (width 0.254) (layer F.Cu) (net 3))
 (segment (start 93.345 46.99) (end 94.6306 48.2756) (width 0.254) (layer F.Cu) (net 3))
 (segment (start 111.76 74.93) (end 106.68 74.93) (width 0.4) (layer B.Cu) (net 8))
 (segment (start 99.06 80.376) (end 99.06 80.01) (width 0.254) (layer F.Cu) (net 4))
 (segment (start 95.7208 83.7152) (end 99.06 80.376) (width 0.254) (layer F.Cu) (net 4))
 (segment (start 94.7406 83.7152) (end 95.7208 83.7152) (width 0.254) (layer F.Cu) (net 4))
 (segment (start 88.9074 77.882) (end 94.7406 83.7152) (width 0.254) (layer F.Cu) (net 4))
 (segment (start 88.9074 71.7925) (end 88.9074 77.882) (width 0.254) (layer F.Cu) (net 4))
 (segment (start 88.1316 71.0167) (end 88.9074 71.7925) (width 0.254) (layer F.Cu) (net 4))
 (segment (start 87.1263 71.0167) (end 88.1316 71.0167) (width 0.254) (layer F.Cu) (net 4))
 (segment (start 83.5924 67.4828) (end 87.1263 71.0167) (width 0.254) (layer F.Cu) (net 4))
 (segment (start 83.5924 58.9932) (end 83.5924 67.4828) (width 0.254) (layer F.Cu) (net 4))
 (segment (start 80.7281 56.1289) (end 83.5924 58.9932) (width 0.254) (layer F.Cu) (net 4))
 (segment (start 80.5242 56.1289) (end 80.7281 56.1289) (width 0.254) (layer F.Cu) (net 4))
 (segment (start 79.465 55.0697) (end 80.5242 56.1289) (width 0.254) (layer F.Cu) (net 4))
 (segment (start 79.465 54.1478) (end 79.465 55.0697) (width 0.254) (layer F.Cu) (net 4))
 (segment (start 80.9861 52.6267) (end 79.465 54.1478) (width 0.254) (layer F.Cu) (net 4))
 (segment (start 85.1683 52.6267) (end 80.9861 52.6267) (width 0.254) (layer F.Cu) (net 4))
 (segment (start 90.805 46.99) (end 85.1683 52.6267) (width 0.254) (layer F.Cu) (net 4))
 (segment (start 111.76 80.01) (end 106.68 80.01) (width 0.4) (layer B.Cu) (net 7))
 (segment (start 92.396 79.696) (end 95.25 82.55) (width 0.254) (layer F.Cu) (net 11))
 (segment (start 92.396 73.0098) (end 92.396 79.696) (width 0.254) (layer F.Cu) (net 11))
 (segment (start 88.0694 68.6832) (end 92.396 73.0098) (width 0.254) (layer F.Cu) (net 11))
 (segment (start 87.1528 68.6832) (end 88.0694 68.6832) (width 0.254) (layer F.Cu) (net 11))
 (segment (start 84.9969 66.5273) (end 87.1528 68.6832) (width 0.254) (layer F.Cu) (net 11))
 (segment (start 84.9969 58.9619) (end 84.9969 66.5273) (width 0.254) (layer F.Cu) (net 11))
 (segment (start 80.645 54.61) (end 84.9969 58.9619) (width 0.254) (layer F.Cu) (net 11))
 (segment (start 89.0974 81.0826) (end 87.63 82.55) (width 0.4) (layer B.Cu) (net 18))
 (segment (start 89.0974 64.1133) (end 89.0974 81.0826) (width 0.4) (layer B.Cu) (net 18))
 (segment (start 88.2886 63.3045) (end 89.0974 64.1133) (width 0.4) (layer B.Cu) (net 18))
 (segment (start 83.3805 63.3045) (end 88.2886 63.3045) (width 0.4) (layer B.Cu) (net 18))
 (segment (start 81.915 64.77) (end 83.3805 63.3045) (width 0.4) (layer B.Cu) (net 18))
 (segment (start 93.4822 75.7022) (end 95.25 77.47) (width 0.254) (layer F.Cu) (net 12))
 (segment (start 93.4822 69.6803) (end 93.4822 75.7022) (width 0.254) (layer F.Cu) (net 12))
 (segment (start 89.044 65.2421) (end 93.4822 69.6803) (width 0.254) (layer F.Cu) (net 12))
 (segment (start 89.044 64.0033) (end 89.044 65.2421) (width 0.254) (layer F.Cu) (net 12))
 (segment (start 85.725 60.6843) (end 89.044 64.0033) (width 0.254) (layer F.Cu) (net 12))
 (segment (start 85.725 57.15) (end 85.725 60.6843) (width 0.254) (layer F.Cu) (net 12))
 (segment (start 83.185 54.61) (end 85.725 57.15) (width 0.254) (layer F.Cu) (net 12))
 (segment (start 85.7851 79.3149) (end 87.63 77.47) (width 0.4) (layer B.Cu) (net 17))
 (segment (start 85.7851 81.2347) (end 85.7851 79.3149) (width 0.4) (layer B.Cu) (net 17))
 (segment (start 82.7079 84.3119) (end 85.7851 81.2347) (width 0.4) (layer B.Cu) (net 17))
 (segment (start 81.1972 84.3119) (end 82.7079 84.3119) (width 0.4) (layer B.Cu) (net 17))
 (segment (start 80.154 83.2687) (end 81.1972 84.3119) (width 0.4) (layer B.Cu) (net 17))
 (segment (start 80.154 71.611) (end 80.154 83.2687) (width 0.4) (layer B.Cu) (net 17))
 (segment (start 81.915 69.85) (end 80.154 71.611) (width 0.4) (layer B.Cu) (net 17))
 (segment (start 93.9906 71.1306) (end 95.25 72.39) (width 0.254) (layer F.Cu) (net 13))
 (segment (start 93.9906 68.3833) (end 93.9906 71.1306) (width 0.254) (layer F.Cu) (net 13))
 (segment (start 89.5524 63.9451) (end 93.9906 68.3833) (width 0.254) (layer F.Cu) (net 13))
 (segment (start 89.5524 63.7272) (end 89.5524 63.9451) (width 0.254) (layer F.Cu) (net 13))
 (segment (start 87.3332 61.508) (end 89.5524 63.7272) (width 0.254) (layer F.Cu) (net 13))
 (segment (start 87.3332 56.2182) (end 87.3332 61.508) (width 0.254) (layer F.Cu) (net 13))
 (segment (start 85.725 54.61) (end 87.3332 56.2182) (width 0.254) (layer F.Cu) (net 13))
 (segment (start 85.09 74.93) (end 87.63 72.39) (width 0.4) (layer F.Cu) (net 16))
 (segment (start 81.915 74.93) (end 85.09 74.93) (width 0.4) (layer F.Cu) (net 16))
 (segment (start 93.8569 65.9169) (end 95.25 67.31) (width 0.254) (layer F.Cu) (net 14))
 (segment (start 93.8569 61.7142) (end 93.8569 65.9169) (width 0.254) (layer F.Cu) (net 14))
 (segment (start 93.1183 60.9756) (end 93.8569 61.7142) (width 0.254) (layer F.Cu) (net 14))
 (segment (start 92.3794 60.9756) (end 93.1183 60.9756) (width 0.254) (layer F.Cu) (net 14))
 (segment (start 91.563 60.1592) (end 92.3794 60.9756) (width 0.254) (layer F.Cu) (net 14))
 (segment (start 91.563 56.5906) (end 91.563 60.1592) (width 0.254) (layer F.Cu) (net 14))
 (segment (start 90.7294 55.757) (end 91.563 56.5906) (width 0.254) (layer F.Cu) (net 14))
 (segment (start 89.412 55.757) (end 90.7294 55.757) (width 0.254) (layer F.Cu) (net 14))
 (segment (start 88.265 54.61) (end 89.412 55.757) (width 0.254) (layer F.Cu) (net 14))
 (segment (start 84.9847 69.9553) (end 87.63 67.31) (width 0.4) (layer B.Cu) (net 15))
 (segment (start 84.9847 76.9403) (end 84.9847 69.9553) (width 0.4) (layer B.Cu) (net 15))
 (segment (start 81.915 80.01) (end 84.9847 76.9403) (width 0.4) (layer B.Cu) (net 15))
 (segment (start 111.76 69.85) (end 106.68 69.85) (width 0.4) (layer B.Cu) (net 9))
 (via (at 96.2594 68.3664) (size 0.889) (layers F.Cu B.Cu) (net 22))
 (segment (start 98.5858 66.04) (end 96.2594 68.3664) (width 0.254) (layer B.Cu) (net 22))
 (segment (start 99.4646 66.04) (end 98.5858 66.04) (width 0.254) (layer B.Cu) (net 22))
 (segment (start 101.5985 63.9061) (end 99.4646 66.04) (width 0.254) (layer B.Cu) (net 22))
 (segment (start 101.5985 63.4135) (end 101.5985 63.9061) (width 0.254) (layer B.Cu) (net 22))
 (segment (start 106.7186 58.2934) (end 101.5985 63.4135) (width 0.254) (layer B.Cu) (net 22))
 (segment (start 109.1017 58.2934) (end 106.7186 58.2934) (width 0.254) (layer B.Cu) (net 22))
 (segment (start 112.395 55.0001) (end 109.1017 58.2934) (width 0.254) (layer B.Cu) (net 22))
 (segment (start 112.395 48.26) (end 112.395 55.0001) (width 0.254) (layer B.Cu) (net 22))
 (segment (start 113.665 46.99) (end 112.395 48.26) (width 0.254) (layer B.Cu) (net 22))
 (segment (start 92.71 66.3837) (end 92.71 62.23) (width 0.254) (layer F.Cu) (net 22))
 (segment (start 94.7995 68.4732) (end 92.71 66.3837) (width 0.254) (layer F.Cu) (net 22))
 (segment (start 96.1526 68.4732) (end 94.7995 68.4732) (width 0.254) (layer F.Cu) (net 22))
 (segment (start 96.2594 68.3664) (end 96.1526 68.4732) (width 0.254) (layer F.Cu) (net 22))
 (segment (start 93.857 58.543) (end 92.71 59.69) (width 0.254) (layer B.Cu) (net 23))
 (segment (start 93.857 56.0492) (end 93.857 58.543) (width 0.254) (layer B.Cu) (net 23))
 (segment (start 94.7536 55.1526) (end 93.857 56.0492) (width 0.254) (layer B.Cu) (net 23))
 (segment (start 94.7536 54.1415) (end 94.7536 55.1526) (width 0.254) (layer B.Cu) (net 23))
 (segment (start 95.7557 53.1394) (end 94.7536 54.1415) (width 0.254) (layer B.Cu) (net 23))
 (segment (start 104.9756 53.1394) (end 95.7557 53.1394) (width 0.254) (layer B.Cu) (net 23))
 (segment (start 111.125 46.99) (end 104.9756 53.1394) (width 0.254) (layer B.Cu) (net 23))
 (segment (start 92.1971 56.6371) (end 92.71 57.15) (width 0.254) (layer B.Cu) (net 24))
 (segment (start 92.1971 54.1464) (end 92.1971 56.6371) (width 0.254) (layer B.Cu) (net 24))
 (segment (start 96.6297 49.7138) (end 92.1971 54.1464) (width 0.254) (layer B.Cu) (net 24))
 (segment (start 105.8612 49.7138) (end 96.6297 49.7138) (width 0.254) (layer B.Cu) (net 24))
 (segment (start 108.585 46.99) (end 105.8612 49.7138) (width 0.254) (layer B.Cu) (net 24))
 (segment (start 95.25 57.15) (end 95.25 59.69) (width 0.5) (layer F.Cu) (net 5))
 (segment (start 95.25 59.69) (end 95.25 62.23) (width 0.5) (layer F.Cu) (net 5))
 (segment (start 95.25 62.23) (end 95.25 64.77) (width 0.5) (layer F.Cu) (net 5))
 (segment (start 96.2896 56.1104) (end 95.25 57.15) (width 0.5) (layer B.Cu) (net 5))
 (segment (start 102.0046 56.1104) (end 96.2896 56.1104) (width 0.5) (layer B.Cu) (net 5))
 (segment (start 103.505 54.61) (end 102.0046 56.1104) (width 0.5) (layer B.Cu) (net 5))
 (segment (start 111.6677 62.23) (end 111.76 62.23) (width 0.5) (layer F.Cu) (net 5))
 (segment (start 109.9565 60.5188) (end 111.6677 62.23) (width 0.5) (layer F.Cu) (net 5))
 (segment (start 109.9565 58.9171) (end 109.9565 60.5188) (width 0.5) (layer F.Cu) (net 5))
 (segment (start 111.1012 57.7724) (end 109.9565 58.9171) (width 0.5) (layer F.Cu) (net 5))
 (segment (start 112.6401 57.7724) (end 111.1012 57.7724) (width 0.5) (layer F.Cu) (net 5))
 (segment (start 115.1941 55.2184) (end 112.6401 57.7724) (width 0.5) (layer F.Cu) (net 5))
 (segment (start 115.1941 53.9751) (end 115.1941 55.2184) (width 0.5) (layer F.Cu) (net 5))
 (segment (start 114.3234 53.1044) (end 115.1941 53.9751) (width 0.5) (layer F.Cu) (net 5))
 (segment (start 105.0106 53.1044) (end 114.3234 53.1044) (width 0.5) (layer F.Cu) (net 5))
 (segment (start 103.505 54.61) (end 105.0106 53.1044) (width 0.5) (layer F.Cu) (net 5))
 (segment (start 93.7466 66.2734) (end 95.25 64.77) (width 0.5) (layer B.Cu) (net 5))
 (segment (start 93.7466 83.2156) (end 93.7466 66.2734) (width 0.5) (layer B.Cu) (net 5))
 (segment (start 94.6213 84.0903) (end 93.7466 83.2156) (width 0.5) (layer B.Cu) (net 5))
 (segment (start 97.5197 84.0903) (end 94.6213 84.0903) (width 0.5) (layer B.Cu) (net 5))
 (segment (start 99.06 82.55) (end 97.5197 84.0903) (width 0.5) (layer B.Cu) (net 5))
 (segment (start 99.378 60.007) (end 99.378 60.0075) (width 0.254) (layer F.Cu) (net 21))
 (segment (start 101.6 57.785) (end 99.378 60.007) (width 0.254) (layer F.Cu) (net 21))
 (segment (start 103.3976 55.9874) (end 101.6 57.785) (width 0.254) (layer B.Cu) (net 21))
 (segment (start 107.2076 55.9874) (end 103.3976 55.9874) (width 0.254) (layer B.Cu) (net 21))
 (segment (start 108.585 54.61) (end 107.2076 55.9874) (width 0.254) (layer B.Cu) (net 21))
 (segment (start 107.95 57.785) (end 104.14 57.785) (width 0.254) (layer B.Cu) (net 20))
 (segment (start 111.125 54.61) (end 107.95 57.785) (width 0.254) (layer B.Cu) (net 20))
 (segment (start 100.0125 61.9125) (end 99.378 61.9125) (width 0.254) (layer B.Cu) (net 20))
 (segment (start 104.14 57.785) (end 100.0125 61.9125) (width 0.254) (layer B.Cu) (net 20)))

